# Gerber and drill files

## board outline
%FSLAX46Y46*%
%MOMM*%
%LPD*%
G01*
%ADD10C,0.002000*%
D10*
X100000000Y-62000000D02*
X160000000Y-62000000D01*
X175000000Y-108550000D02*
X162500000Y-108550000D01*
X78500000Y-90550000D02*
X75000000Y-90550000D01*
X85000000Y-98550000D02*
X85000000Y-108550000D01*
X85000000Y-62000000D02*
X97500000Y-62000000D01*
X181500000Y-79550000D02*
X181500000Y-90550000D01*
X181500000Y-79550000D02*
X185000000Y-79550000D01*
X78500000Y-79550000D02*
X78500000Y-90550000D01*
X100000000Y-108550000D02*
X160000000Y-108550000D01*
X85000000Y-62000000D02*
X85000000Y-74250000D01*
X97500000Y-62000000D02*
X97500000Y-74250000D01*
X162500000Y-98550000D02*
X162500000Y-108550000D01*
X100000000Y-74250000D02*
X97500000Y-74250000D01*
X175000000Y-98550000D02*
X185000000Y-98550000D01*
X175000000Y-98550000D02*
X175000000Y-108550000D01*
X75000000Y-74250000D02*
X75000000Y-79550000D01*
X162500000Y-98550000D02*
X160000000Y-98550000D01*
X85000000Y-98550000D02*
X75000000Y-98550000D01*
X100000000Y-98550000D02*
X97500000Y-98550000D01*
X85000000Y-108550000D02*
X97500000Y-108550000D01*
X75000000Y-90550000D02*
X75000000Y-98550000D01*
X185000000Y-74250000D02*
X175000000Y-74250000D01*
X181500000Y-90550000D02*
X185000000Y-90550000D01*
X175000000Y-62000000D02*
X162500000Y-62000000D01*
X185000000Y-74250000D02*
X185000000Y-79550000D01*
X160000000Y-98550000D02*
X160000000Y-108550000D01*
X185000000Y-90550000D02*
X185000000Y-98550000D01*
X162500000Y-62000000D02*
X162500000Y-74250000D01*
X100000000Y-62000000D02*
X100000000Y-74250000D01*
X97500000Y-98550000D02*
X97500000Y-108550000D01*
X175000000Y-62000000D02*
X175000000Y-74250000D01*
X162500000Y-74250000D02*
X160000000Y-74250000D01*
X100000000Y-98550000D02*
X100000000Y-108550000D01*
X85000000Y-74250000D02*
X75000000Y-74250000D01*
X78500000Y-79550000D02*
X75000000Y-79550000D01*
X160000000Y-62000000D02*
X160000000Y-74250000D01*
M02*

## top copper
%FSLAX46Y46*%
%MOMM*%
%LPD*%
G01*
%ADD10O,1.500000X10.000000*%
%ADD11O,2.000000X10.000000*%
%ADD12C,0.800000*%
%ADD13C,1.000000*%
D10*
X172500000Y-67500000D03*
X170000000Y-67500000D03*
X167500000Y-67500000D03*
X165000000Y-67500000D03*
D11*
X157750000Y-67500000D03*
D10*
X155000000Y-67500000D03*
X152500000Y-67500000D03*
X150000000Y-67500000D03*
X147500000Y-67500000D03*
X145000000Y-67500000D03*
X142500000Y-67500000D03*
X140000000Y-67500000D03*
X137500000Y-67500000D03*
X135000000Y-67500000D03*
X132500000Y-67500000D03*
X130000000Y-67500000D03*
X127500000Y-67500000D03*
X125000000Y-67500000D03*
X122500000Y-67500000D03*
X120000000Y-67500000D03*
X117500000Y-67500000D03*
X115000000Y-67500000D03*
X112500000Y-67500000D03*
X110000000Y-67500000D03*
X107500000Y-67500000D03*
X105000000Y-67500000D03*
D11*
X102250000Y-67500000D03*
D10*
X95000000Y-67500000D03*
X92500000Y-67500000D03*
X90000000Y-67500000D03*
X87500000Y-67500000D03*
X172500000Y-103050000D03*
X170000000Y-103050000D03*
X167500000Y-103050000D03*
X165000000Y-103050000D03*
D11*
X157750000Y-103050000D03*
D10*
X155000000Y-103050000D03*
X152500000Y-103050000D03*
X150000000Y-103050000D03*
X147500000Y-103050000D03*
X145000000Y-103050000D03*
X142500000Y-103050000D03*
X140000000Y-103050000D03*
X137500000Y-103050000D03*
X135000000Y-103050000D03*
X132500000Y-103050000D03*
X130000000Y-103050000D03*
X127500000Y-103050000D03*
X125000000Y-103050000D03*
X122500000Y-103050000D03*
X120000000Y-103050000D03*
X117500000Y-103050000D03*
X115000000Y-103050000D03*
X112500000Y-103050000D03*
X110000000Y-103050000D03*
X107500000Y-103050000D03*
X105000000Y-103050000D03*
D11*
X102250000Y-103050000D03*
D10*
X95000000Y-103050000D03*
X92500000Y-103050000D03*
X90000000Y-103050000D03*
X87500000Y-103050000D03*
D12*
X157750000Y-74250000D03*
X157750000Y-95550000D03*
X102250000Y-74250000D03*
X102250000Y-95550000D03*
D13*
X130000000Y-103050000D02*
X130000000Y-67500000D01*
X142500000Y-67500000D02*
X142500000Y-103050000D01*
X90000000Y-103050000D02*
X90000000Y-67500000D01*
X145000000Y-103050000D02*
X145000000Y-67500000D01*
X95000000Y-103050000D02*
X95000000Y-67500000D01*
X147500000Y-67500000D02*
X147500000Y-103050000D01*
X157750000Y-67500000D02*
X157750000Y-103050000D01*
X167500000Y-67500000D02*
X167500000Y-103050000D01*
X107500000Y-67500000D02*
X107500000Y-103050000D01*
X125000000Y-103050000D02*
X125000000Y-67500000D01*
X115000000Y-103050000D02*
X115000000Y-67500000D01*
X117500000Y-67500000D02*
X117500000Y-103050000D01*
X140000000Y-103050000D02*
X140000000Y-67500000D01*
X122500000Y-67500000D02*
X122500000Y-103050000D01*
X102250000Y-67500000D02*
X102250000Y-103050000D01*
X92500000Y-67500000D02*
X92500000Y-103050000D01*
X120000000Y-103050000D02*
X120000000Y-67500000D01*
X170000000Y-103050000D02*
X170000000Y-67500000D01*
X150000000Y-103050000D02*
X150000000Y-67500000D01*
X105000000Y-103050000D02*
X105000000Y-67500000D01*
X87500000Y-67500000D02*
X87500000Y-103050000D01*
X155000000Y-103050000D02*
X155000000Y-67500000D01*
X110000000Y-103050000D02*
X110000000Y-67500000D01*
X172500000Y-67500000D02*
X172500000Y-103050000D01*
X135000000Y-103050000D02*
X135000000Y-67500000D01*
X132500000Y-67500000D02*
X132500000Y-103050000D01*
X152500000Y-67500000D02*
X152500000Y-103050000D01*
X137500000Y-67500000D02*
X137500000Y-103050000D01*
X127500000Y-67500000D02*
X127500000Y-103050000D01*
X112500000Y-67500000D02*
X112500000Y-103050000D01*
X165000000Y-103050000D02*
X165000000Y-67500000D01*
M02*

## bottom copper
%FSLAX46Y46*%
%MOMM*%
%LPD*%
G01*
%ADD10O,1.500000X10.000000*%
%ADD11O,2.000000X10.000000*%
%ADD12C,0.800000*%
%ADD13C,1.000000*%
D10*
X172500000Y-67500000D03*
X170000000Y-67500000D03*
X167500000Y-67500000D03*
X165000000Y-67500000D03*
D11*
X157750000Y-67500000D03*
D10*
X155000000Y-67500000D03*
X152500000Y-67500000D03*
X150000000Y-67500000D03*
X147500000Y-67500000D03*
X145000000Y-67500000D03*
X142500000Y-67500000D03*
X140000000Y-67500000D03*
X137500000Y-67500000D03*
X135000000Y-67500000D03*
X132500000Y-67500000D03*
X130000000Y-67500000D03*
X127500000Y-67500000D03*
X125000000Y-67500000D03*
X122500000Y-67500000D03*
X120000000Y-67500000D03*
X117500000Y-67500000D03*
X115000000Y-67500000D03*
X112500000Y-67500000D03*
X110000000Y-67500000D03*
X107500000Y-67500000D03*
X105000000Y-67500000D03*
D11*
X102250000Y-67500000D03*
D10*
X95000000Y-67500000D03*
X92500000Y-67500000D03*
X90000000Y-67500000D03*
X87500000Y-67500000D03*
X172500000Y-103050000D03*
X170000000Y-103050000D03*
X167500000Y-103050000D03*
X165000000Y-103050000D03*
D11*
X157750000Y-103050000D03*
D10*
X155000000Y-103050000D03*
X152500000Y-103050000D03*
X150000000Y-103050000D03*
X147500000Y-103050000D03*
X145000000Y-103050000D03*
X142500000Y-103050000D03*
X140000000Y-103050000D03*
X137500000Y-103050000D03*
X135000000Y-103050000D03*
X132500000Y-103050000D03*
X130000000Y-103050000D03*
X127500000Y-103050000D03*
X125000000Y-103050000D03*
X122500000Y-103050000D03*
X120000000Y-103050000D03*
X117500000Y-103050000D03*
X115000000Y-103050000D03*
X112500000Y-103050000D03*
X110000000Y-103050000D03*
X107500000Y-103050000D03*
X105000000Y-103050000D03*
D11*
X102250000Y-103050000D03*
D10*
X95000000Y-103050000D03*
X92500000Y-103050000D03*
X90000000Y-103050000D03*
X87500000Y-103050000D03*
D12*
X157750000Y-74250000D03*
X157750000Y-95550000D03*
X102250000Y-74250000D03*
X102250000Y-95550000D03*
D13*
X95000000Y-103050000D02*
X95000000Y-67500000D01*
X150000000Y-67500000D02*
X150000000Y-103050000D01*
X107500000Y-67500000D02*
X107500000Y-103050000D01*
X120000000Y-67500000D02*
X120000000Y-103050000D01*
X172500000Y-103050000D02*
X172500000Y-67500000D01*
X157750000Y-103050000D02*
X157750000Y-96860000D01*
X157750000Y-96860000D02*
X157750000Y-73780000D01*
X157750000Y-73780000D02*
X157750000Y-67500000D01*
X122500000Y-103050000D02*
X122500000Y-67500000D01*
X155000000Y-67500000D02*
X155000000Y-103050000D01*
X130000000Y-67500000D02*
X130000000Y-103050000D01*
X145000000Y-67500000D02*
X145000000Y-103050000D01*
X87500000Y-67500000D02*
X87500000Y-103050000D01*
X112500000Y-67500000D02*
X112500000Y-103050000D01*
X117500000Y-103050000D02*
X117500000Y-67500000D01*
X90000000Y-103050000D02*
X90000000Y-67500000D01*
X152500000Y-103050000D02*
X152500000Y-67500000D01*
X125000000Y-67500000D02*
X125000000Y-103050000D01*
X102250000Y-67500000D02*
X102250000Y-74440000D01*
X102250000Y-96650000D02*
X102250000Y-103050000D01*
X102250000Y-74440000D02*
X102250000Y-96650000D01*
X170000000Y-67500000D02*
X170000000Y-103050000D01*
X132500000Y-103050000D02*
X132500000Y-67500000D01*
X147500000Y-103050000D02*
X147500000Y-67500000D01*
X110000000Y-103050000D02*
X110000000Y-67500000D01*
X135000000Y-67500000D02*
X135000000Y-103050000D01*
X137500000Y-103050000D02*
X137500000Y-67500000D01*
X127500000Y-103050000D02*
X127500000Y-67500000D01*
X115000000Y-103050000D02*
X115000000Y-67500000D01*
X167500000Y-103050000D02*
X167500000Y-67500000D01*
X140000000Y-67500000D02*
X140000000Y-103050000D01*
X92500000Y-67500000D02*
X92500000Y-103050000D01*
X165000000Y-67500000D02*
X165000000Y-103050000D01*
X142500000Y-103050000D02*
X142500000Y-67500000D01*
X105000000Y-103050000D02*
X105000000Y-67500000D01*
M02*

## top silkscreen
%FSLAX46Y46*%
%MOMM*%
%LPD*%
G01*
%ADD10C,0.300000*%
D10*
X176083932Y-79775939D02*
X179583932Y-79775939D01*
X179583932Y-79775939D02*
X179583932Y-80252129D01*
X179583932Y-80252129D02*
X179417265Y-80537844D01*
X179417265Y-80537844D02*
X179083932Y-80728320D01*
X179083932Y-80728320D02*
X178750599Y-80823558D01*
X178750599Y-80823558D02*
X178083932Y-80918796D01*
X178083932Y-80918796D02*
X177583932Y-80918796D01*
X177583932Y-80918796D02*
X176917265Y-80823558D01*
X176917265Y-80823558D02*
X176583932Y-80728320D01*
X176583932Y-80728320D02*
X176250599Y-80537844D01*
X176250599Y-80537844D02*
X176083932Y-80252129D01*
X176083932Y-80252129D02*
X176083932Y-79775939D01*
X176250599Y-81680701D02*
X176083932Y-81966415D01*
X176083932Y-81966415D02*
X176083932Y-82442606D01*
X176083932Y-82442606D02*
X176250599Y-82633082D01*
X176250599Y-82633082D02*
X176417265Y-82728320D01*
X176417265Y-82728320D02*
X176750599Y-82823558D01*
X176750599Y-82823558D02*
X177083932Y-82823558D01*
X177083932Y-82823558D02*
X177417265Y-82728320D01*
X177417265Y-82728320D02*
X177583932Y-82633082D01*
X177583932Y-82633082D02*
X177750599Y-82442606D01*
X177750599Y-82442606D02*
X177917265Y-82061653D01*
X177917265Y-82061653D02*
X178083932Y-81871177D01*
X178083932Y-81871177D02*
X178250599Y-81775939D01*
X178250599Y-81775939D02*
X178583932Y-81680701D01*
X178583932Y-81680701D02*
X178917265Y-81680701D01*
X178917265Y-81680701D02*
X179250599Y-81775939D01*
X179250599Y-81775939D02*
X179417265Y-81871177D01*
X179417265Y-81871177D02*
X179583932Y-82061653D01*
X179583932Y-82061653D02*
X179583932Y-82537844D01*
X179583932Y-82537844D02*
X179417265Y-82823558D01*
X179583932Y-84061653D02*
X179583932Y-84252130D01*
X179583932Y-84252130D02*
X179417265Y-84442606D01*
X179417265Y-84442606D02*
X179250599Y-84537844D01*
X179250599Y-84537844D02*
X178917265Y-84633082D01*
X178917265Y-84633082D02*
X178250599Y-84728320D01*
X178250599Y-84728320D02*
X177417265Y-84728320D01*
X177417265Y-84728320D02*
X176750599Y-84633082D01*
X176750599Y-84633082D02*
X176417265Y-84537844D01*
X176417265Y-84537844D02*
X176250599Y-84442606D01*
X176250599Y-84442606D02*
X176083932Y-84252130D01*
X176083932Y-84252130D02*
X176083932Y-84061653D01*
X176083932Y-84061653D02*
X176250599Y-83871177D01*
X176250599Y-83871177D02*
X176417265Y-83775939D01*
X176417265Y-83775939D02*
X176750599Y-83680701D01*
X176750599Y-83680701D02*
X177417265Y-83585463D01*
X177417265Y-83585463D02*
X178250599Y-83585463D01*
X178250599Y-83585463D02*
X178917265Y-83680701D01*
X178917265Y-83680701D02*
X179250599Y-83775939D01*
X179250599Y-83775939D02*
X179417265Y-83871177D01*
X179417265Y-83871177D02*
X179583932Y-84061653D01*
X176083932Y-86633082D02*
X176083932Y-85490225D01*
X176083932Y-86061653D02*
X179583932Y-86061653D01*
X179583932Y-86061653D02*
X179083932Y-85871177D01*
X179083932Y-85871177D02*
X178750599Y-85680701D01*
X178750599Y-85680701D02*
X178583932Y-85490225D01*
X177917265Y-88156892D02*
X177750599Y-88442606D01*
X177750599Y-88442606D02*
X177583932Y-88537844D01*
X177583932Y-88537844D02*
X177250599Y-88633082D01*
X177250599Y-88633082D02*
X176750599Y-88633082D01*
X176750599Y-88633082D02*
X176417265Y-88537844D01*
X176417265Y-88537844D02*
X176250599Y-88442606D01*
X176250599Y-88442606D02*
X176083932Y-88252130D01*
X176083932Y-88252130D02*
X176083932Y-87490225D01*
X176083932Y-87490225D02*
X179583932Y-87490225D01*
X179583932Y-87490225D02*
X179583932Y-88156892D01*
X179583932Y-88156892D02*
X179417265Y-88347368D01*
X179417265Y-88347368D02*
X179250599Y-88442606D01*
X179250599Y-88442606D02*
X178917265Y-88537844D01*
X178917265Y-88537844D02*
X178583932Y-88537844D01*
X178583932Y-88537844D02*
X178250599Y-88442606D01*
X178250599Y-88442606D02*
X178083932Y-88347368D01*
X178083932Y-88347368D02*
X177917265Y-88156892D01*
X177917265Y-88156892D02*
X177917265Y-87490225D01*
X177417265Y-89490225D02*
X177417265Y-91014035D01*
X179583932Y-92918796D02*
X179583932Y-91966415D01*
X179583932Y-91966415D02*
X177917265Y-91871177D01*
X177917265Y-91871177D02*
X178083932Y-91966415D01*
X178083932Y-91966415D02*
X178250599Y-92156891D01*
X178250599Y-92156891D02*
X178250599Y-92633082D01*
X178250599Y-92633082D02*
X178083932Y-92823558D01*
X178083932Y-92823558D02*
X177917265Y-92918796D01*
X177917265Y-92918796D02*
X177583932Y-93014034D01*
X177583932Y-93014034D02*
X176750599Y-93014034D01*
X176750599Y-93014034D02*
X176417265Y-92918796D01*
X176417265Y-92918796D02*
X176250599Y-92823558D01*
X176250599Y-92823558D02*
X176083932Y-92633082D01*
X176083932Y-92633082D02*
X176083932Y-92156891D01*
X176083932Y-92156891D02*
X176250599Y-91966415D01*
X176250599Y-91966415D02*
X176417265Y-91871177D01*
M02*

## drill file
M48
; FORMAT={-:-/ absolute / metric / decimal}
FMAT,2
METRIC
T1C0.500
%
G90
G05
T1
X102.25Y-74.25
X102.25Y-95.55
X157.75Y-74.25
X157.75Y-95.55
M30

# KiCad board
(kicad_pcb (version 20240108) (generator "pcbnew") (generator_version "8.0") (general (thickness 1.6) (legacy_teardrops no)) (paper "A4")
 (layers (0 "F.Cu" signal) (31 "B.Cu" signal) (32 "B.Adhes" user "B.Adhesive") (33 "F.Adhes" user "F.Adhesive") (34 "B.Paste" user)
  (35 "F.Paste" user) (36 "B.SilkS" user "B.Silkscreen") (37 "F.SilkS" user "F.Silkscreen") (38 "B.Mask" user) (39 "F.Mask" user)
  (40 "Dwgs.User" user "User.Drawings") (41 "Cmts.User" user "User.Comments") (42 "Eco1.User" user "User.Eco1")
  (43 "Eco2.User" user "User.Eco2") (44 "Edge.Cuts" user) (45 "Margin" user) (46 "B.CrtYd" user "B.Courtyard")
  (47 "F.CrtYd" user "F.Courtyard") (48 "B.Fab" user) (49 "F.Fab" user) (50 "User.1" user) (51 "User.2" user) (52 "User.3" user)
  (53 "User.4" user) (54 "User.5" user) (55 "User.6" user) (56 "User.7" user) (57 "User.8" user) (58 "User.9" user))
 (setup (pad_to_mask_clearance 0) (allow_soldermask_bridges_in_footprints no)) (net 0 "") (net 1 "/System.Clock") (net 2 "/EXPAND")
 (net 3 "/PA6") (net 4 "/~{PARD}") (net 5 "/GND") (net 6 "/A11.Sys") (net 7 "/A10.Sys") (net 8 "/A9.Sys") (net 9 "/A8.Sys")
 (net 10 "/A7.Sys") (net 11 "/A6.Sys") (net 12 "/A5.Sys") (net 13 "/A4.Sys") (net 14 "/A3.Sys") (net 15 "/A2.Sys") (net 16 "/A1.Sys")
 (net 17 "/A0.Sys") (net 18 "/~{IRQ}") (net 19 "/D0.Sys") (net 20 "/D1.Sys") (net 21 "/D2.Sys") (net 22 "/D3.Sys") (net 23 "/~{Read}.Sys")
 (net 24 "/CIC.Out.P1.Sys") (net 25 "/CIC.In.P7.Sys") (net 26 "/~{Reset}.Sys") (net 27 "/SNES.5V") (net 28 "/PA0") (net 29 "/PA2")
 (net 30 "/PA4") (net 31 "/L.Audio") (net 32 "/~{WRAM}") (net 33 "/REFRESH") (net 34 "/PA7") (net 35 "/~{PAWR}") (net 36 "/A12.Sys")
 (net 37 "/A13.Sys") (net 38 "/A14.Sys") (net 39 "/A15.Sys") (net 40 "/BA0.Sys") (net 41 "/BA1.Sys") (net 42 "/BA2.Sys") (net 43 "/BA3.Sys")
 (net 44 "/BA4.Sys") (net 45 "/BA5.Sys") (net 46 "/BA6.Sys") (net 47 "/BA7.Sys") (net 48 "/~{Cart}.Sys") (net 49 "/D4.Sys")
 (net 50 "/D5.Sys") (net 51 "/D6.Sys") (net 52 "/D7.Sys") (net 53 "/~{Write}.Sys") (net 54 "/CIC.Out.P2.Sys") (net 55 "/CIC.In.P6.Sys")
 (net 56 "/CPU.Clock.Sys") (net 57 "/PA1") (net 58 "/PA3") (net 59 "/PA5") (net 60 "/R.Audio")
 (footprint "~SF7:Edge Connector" (layer "F.Cu") (at 130 67.5)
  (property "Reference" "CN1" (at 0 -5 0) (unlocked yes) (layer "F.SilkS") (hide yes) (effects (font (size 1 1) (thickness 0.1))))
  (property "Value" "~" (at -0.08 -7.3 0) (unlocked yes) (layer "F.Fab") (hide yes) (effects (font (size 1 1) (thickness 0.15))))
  (pad "1" smd oval (at 42.5 0) (size 1.5 10) (layers "B.Cu" "B.Mask") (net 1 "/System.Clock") (thermal_bridge_angle 45))
  (pad "2" smd oval (at 40 0) (size 1.5 10) (layers "B.Cu" "B.Mask") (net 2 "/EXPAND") (thermal_bridge_angle 45))
  (pad "3" smd oval (at 37.5 0) (size 1.5 10) (layers "B.Cu" "B.Mask") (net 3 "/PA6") (thermal_bridge_angle 45))
  (pad "4" smd oval (at 35 0) (size 1.5 10) (layers "B.Cu" "B.Mask") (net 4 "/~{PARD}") (thermal_bridge_angle 45))
  (pad "5" smd oval (at 27.75 0) (size 2 10) (layers "B.Cu" "B.Mask") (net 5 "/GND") (thermal_bridge_angle 45))
  (pad "6" smd oval (at 25 0) (size 1.5 10) (layers "B.Cu" "B.Mask") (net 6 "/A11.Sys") (thermal_bridge_angle 45))
  (pad "7" smd oval (at 22.5 0) (size 1.5 10) (layers "B.Cu" "B.Mask") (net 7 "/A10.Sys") (thermal_bridge_angle 45))
  (pad "8" smd oval (at 20 0) (size 1.5 10) (layers "B.Cu" "B.Mask") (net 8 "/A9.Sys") (thermal_bridge_angle 45))
  (pad "9" smd oval (at 17.5 0) (size 1.5 10) (layers "B.Cu" "B.Mask") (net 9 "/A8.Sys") (thermal_bridge_angle 45))
  (pad "10" smd oval (at 15 0) (size 1.5 10) (layers "B.Cu" "B.Mask") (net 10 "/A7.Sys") (thermal_bridge_angle 45))
  (pad "11" smd oval (at 12.5 0) (size 1.5 10) (layers "B.Cu" "B.Mask") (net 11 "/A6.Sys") (thermal_bridge_angle 45))
  (pad "12" smd oval (at 10 0) (size 1.5 10) (layers "B.Cu" "B.Mask") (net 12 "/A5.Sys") (thermal_bridge_angle 45))
  (pad "13" smd oval (at 7.5 0) (size 1.5 10) (layers "B.Cu" "B.Mask") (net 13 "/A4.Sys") (thermal_bridge_angle 45))
  (pad "14" smd oval (at 5 0) (size 1.5 10) (layers "B.Cu" "B.Mask") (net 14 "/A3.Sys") (thermal_bridge_angle 45))
  (pad "15" smd oval (at 2.5 0) (size 1.5 10) (layers "B.Cu" "B.Mask") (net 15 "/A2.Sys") (thermal_bridge_angle 45))
  (pad "16" smd oval (at 0 0) (size 1.5 10) (layers "B.Cu" "B.Mask") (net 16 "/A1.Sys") (thermal_bridge_angle 45))
  (pad "17" smd oval (at -2.5 0) (size 1.5 10) (layers "B.Cu" "B.Mask") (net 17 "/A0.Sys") (thermal_bridge_angle 45))
  (pad "18" smd oval (at -5 0) (size 1.5 10) (layers "B.Cu" "B.Mask") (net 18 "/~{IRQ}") (thermal_bridge_angle 45))
  (pad "19" smd oval (at -7.5 0) (size 1.5 10) (layers "B.Cu" "B.Mask") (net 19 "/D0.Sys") (thermal_bridge_angle 45))
  (pad "20" smd oval (at -10 0) (size 1.5 10) (layers "B.Cu" "B.Mask") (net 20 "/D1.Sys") (thermal_bridge_angle 45))
  (pad "21" smd oval (at -12.5 0) (size 1.5 10) (layers "B.Cu" "B.Mask") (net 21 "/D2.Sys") (thermal_bridge_angle 45))
  (pad "22" smd oval (at -15 0) (size 1.5 10) (layers "B.Cu" "B.Mask") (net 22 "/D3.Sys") (thermal_bridge_angle 45))
  (pad "23" smd oval (at -17.5 0) (size 1.5 10) (layers "B.Cu" "B.Mask") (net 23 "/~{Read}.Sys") (thermal_bridge_angle 45))
  (pad "24" smd oval (at -20 0) (size 1.5 10) (layers "B.Cu" "B.Mask") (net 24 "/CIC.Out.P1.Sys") (thermal_bridge_angle 45))
  (pad "25" smd oval (at -22.5 0) (size 1.5 10) (layers "B.Cu" "B.Mask") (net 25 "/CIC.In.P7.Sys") (thermal_bridge_angle 45))
  (pad "26" smd oval (at -25 0) (size 1.5 10) (layers "B.Cu" "B.Mask") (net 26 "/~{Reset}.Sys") (thermal_bridge_angle 45))
  (pad "27" smd oval (at -27.75 0) (size 2 10) (layers "B.Cu" "B.Mask") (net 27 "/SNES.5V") (thermal_bridge_angle 45))
  (pad "28" smd oval (at -35 0) (size 1.5 10) (layers "B.Cu" "B.Mask") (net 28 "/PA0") (thermal_bridge_angle 45))
  (pad "29" smd oval (at -37.5 0) (size 1.5 10) (layers "B.Cu" "B.Mask") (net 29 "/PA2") (thermal_bridge_angle 45))
  (pad "30" smd oval (at -40 0) (size 1.5 10) (layers "B.Cu" "B.Mask") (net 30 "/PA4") (thermal_bridge_angle 45))
  (pad "31" smd oval (at -42.5 0) (size 1.5 10) (layers "B.Cu" "B.Mask") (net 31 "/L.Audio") (thermal_bridge_angle 45))
  (pad "32" smd oval (at 42.5 0) (size 1.5 10) (layers "F.Cu" "F.Mask") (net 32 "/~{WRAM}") (thermal_bridge_angle 45))
  (pad "33" smd oval (at 40 0) (size 1.5 10) (layers "F.Cu" "F.Mask") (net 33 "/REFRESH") (thermal_bridge_angle 45))
  (pad "34" smd oval (at 37.5 0) (size 1.5 10) (layers "F.Cu" "F.Mask") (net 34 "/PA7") (thermal_bridge_angle 45))
  (pad "35" smd oval (at 35 0) (size 1.5 10) (layers "F.Cu" "F.Mask") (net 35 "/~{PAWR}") (thermal_bridge_angle 45))
  (pad "36" smd oval (at 27.75 0) (size 2 10) (layers "F.Cu" "F.Mask") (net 5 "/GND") (thermal_bridge_angle 45))
  (pad "37" smd oval (at 25 0) (size 1.5 10) (layers "F.Cu" "F.Mask") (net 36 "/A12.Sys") (thermal_bridge_angle 45))
  (pad "38" smd oval (at 22.5 0) (size 1.5 10) (layers "F.Cu" "F.Mask") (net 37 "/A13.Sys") (thermal_bridge_angle 45))
  (pad "39" smd oval (at 20 0) (size 1.5 10) (layers "F.Cu" "F.Mask") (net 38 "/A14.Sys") (thermal_bridge_angle 45))
  (pad "40" smd oval (at 17.5 0) (size 1.5 10) (layers "F.Cu" "F.Mask") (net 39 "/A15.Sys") (thermal_bridge_angle 45))
  (pad "41" smd oval (at 15 0) (size 1.5 10) (layers "F.Cu" "F.Mask") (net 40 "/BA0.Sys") (thermal_bridge_angle 45))
  (pad "42" smd oval (at 12.5 0) (size 1.5 10) (layers "F.Cu" "F.Mask") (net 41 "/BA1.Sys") (thermal_bridge_angle 45))
  (pad "43" smd oval (at 10 0) (size 1.5 10) (layers "F.Cu" "F.Mask") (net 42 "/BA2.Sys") (thermal_bridge_angle 45))
  (pad "44" smd oval (at 7.5 0) (size 1.5 10) (layers "F.Cu" "F.Mask") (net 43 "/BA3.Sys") (thermal_bridge_angle 45))
  (pad "45" smd oval (at 5 0) (size 1.5 10) (layers "F.Cu" "F.Mask") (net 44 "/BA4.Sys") (thermal_bridge_angle 45))
  (pad "46" smd oval (at 2.5 0) (size 1.5 10) (layers "F.Cu" "F.Mask") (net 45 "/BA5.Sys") (thermal_bridge_angle 45))
  (pad "47" smd oval (at 0 0) (size 1.5 10) (layers "F.Cu" "F.Mask") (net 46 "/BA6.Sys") (thermal_bridge_angle 45))
  (pad "48" smd oval (at -2.5 0) (size 1.5 10) (layers "F.Cu" "F.Mask") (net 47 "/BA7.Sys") (thermal_bridge_angle 45))
  (pad "49" smd oval (at -5 0) (size 1.5 10) (layers "F.Cu" "F.Mask") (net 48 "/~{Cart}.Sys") (thermal_bridge_angle 45))
  (pad "50" smd oval (at -7.5 0) (size 1.5 10) (layers "F.Cu" "F.Mask") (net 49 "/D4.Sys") (thermal_bridge_angle 45))
  (pad "51" smd oval (at -10 0) (size 1.5 10) (layers "F.Cu" "F.Mask") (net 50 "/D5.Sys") (thermal_bridge_angle 45))
  (pad "52" smd oval (at -12.5 0) (size 1.5 10) (layers "F.Cu" "F.Mask") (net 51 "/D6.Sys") (thermal_bridge_angle 45))
  (pad "53" smd oval (at -15 0) (size 1.5 10) (layers "F.Cu" "F.Mask") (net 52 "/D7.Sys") (thermal_bridge_angle 45))
  (pad "54" smd oval (at -17.5 0) (size 1.5 10) (layers "F.Cu" "F.Mask") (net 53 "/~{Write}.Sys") (thermal_bridge_angle 45))
  (pad "55" smd oval (at -20 0) (size 1.5 10) (layers "F.Cu" "F.Mask") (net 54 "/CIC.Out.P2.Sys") (thermal_bridge_angle 45))
  (pad "56" smd oval (at -22.5 0) (size 1.5 10) (layers "F.Cu" "F.Mask") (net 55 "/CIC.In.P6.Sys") (thermal_bridge_angle 45))
  (pad "57" smd oval (at -25 0) (size 1.5 10) (layers "F.Cu" "F.Mask") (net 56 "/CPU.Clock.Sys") (thermal_bridge_angle 45))
  (pad "58" smd oval (at -27.75 0) (size 2 10) (layers "F.Cu" "F.Mask") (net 27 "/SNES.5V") (thermal_bridge_angle 45))
  (pad "59" smd oval (at -35 0) (size 1.5 10) (layers "F.Cu" "F.Mask") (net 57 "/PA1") (thermal_bridge_angle 45))
  (pad "60" smd oval (at -37.5 0) (size 1.5 10) (layers "F.Cu" "F.Mask") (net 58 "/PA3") (thermal_bridge_angle 45))
  (pad "61" smd oval (at -40 0) (size 1.5 10) (layers "F.Cu" "F.Mask") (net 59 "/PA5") (thermal_bridge_angle 45))
  (pad "62" smd oval (at -42.5 0) (size 1.5 10) (layers "F.Cu" "F.Mask") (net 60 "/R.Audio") (thermal_bridge_angle 45)))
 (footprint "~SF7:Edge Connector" (layer "F.Cu") (at 130 103.05)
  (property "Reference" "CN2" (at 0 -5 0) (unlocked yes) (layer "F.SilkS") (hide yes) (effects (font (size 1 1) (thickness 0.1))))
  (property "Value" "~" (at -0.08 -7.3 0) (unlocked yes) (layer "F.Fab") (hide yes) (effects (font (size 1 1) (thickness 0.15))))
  (pad "1" smd oval (at 42.5 0) (size 1.5 10) (layers "B.Cu" "B.Mask") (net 1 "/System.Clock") (thermal_bridge_angle 45))
  (pad "2" smd oval (at 40 0) (size 1.5 10) (layers "B.Cu" "B.Mask") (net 2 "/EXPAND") (thermal_bridge_angle 45))
  (pad "3" smd oval (at 37.5 0) (size 1.5 10) (layers "B.Cu" "B.Mask") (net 3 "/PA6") (thermal_bridge_angle 45))
  (pad "4" smd oval (at 35 0) (size 1.5 10) (layers "B.Cu" "B.Mask") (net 4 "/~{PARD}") (thermal_bridge_angle 45))
  (pad "5" smd oval (at 27.75 0) (size 2 10) (layers "B.Cu" "B.Mask") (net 5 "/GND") (thermal_bridge_angle 45))
  (pad "6" smd oval (at 25 0) (size 1.5 10) (layers "B.Cu" "B.Mask") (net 6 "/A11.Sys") (thermal_bridge_angle 45))
  (pad "7" smd oval (at 22.5 0) (size 1.5 10) (layers "B.Cu" "B.Mask") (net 7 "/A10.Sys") (thermal_bridge_angle 45))
  (pad "8" smd oval (at 20 0) (size 1.5 10) (layers "B.Cu" "B.Mask") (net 8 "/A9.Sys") (thermal_bridge_angle 45))
  (pad "9" smd oval (at 17.5 0) (size 1.5 10) (layers "B.Cu" "B.Mask") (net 9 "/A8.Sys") (thermal_bridge_angle 45))
  (pad "10" smd oval (at 15 0) (size 1.5 10) (layers "B.Cu" "B.Mask") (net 10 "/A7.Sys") (thermal_bridge_angle 45))
  (pad "11" smd oval (at 12.5 0) (size 1.5 10) (layers "B.Cu" "B.Mask") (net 11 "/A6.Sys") (thermal_bridge_angle 45))
  (pad "12" smd oval (at 10 0) (size 1.5 10) (layers "B.Cu" "B.Mask") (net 12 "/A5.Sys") (thermal_bridge_angle 45))
  (pad "13" smd oval (at 7.5 0) (size 1.5 10) (layers "B.Cu" "B.Mask") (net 13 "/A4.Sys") (thermal_bridge_angle 45))
  (pad "14" smd oval (at 5 0) (size 1.5 10) (layers "B.Cu" "B.Mask") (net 14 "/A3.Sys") (thermal_bridge_angle 45))
  (pad "15" smd oval (at 2.5 0) (size 1.5 10) (layers "B.Cu" "B.Mask") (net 15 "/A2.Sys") (thermal_bridge_angle 45))
  (pad "16" smd oval (at 0 0) (size 1.5 10) (layers "B.Cu" "B.Mask") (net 16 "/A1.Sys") (thermal_bridge_angle 45))
  (pad "17" smd oval (at -2.5 0) (size 1.5 10) (layers "B.Cu" "B.Mask") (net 17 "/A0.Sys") (thermal_bridge_angle 45))
  (pad "18" smd oval (at -5 0) (size 1.5 10) (layers "B.Cu" "B.Mask") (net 18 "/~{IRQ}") (thermal_bridge_angle 45))
  (pad "19" smd oval (at -7.5 0) (size 1.5 10) (layers "B.Cu" "B.Mask") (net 19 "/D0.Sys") (thermal_bridge_angle 45))
  (pad "20" smd oval (at -10 0) (size 1.5 10) (layers "B.Cu" "B.Mask") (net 20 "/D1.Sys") (thermal_bridge_angle 45))
  (pad "21" smd oval (at -12.5 0) (size 1.5 10) (layers "B.Cu" "B.Mask") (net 21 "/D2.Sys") (thermal_bridge_angle 45))
  (pad "22" smd oval (at -15 0) (size 1.5 10) (layers "B.Cu" "B.Mask") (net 22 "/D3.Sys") (thermal_bridge_angle 45))
  (pad "23" smd oval (at -17.5 0) (size 1.5 10) (layers "B.Cu" "B.Mask") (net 23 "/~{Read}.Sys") (thermal_bridge_angle 45))
  (pad "24" smd oval (at -20 0) (size 1.5 10) (layers "B.Cu" "B.Mask") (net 24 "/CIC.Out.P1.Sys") (thermal_bridge_angle 45))
  (pad "25" smd oval (at -22.5 0) (size 1.5 10) (layers "B.Cu" "B.Mask") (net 25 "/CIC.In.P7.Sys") (thermal_bridge_angle 45))
  (pad "26" smd oval (at -25 0) (size 1.5 10) (layers "B.Cu" "B.Mask") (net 26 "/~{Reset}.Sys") (thermal_bridge_angle 45))
  (pad "27" smd oval (at -27.75 0) (size 2 10) (layers "B.Cu" "B.Mask") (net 27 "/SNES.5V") (thermal_bridge_angle 45))
  (pad "28" smd oval (at -35 0) (size 1.5 10) (layers "B.Cu" "B.Mask") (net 28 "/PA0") (thermal_bridge_angle 45))
  (pad "29" smd oval (at -37.5 0) (size 1.5 10) (layers "B.Cu" "B.Mask") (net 29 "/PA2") (thermal_bridge_angle 45))
  (pad "30" smd oval (at -40 0) (size 1.5 10) (layers "B.Cu" "B.Mask") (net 30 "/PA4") (thermal_bridge_angle 45))
  (pad "31" smd oval (at -42.5 0) (size 1.5 10) (layers "B.Cu" "B.Mask") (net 31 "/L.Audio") (thermal_bridge_angle 45))
  (pad "32" smd oval (at 42.5 0) (size 1.5 10) (layers "F.Cu" "F.Mask") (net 32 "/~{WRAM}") (thermal_bridge_angle 45))
  (pad "33" smd oval (at 40 0) (size 1.5 10) (layers "F.Cu" "F.Mask") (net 33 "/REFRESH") (thermal_bridge_angle 45))
  (pad "34" smd oval (at 37.5 0) (size 1.5 10) (layers "F.Cu" "F.Mask") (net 34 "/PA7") (thermal_bridge_angle 45))
  (pad "35" smd oval (at 35 0) (size 1.5 10) (layers "F.Cu" "F.Mask") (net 35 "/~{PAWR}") (thermal_bridge_angle 45))
  (pad "36" smd oval (at 27.75 0) (size 2 10) (layers "F.Cu" "F.Mask") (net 5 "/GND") (thermal_bridge_angle 45))
  (pad "37" smd oval (at 25 0) (size 1.5 10) (layers "F.Cu" "F.Mask") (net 36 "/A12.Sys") (thermal_bridge_angle 45))
  (pad "38" smd oval (at 22.5 0) (size 1.5 10) (layers "F.Cu" "F.Mask") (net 37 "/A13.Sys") (thermal_bridge_angle 45))
  (pad "39" smd oval (at 20 0) (size 1.5 10) (layers "F.Cu" "F.Mask") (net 38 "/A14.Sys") (thermal_bridge_angle 45))
  (pad "40" smd oval (at 17.5 0) (size 1.5 10) (layers "F.Cu" "F.Mask") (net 39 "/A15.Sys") (thermal_bridge_angle 45))
  (pad "41" smd oval (at 15 0) (size 1.5 10) (layers "F.Cu" "F.Mask") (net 40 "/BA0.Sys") (thermal_bridge_angle 45))
  (pad "42" smd oval (at 12.5 0) (size 1.5 10) (layers "F.Cu" "F.Mask") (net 41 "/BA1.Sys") (thermal_bridge_angle 45))
  (pad "43" smd oval (at 10 0) (size 1.5 10) (layers "F.Cu" "F.Mask") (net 42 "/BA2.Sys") (thermal_bridge_angle 45))
  (pad "44" smd oval (at 7.5 0) (size 1.5 10) (layers "F.Cu" "F.Mask") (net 43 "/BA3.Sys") (thermal_bridge_angle 45))
  (pad "45" smd oval (at 5 0) (size 1.5 10) (layers "F.Cu" "F.Mask") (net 44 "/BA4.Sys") (thermal_bridge_angle 45))
  (pad "46" smd oval (at 2.5 0) (size 1.5 10) (layers "F.Cu" "F.Mask") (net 45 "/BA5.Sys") (thermal_bridge_angle 45))
  (pad "47" smd oval (at 0 0) (size 1.5 10) (layers "F.Cu" "F.Mask") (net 46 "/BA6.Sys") (thermal_bridge_angle 45))
  (pad "48" smd oval (at -2.5 0) (size 1.5 10) (layers "F.Cu" "F.Mask") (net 47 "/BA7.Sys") (thermal_bridge_angle 45))
  (pad "49" smd oval (at -5 0) (size 1.5 10) (layers "F.Cu" "F.Mask") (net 48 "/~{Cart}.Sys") (thermal_bridge_angle 45))
  (pad "50" smd oval (at -7.5 0) (size 1.5 10) (layers "F.Cu" "F.Mask") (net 49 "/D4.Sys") (thermal_bridge_angle 45))
  (pad "51" smd oval (at -10 0) (size 1.5 10) (layers "F.Cu" "F.Mask") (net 50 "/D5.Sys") (thermal_bridge_angle 45))
  (pad "52" smd oval (at -12.5 0) (size 1.5 10) (layers "F.Cu" "F.Mask") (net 51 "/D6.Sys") (thermal_bridge_angle 45))
  (pad "53" smd oval (at -15 0) (size 1.5 10) (layers "F.Cu" "F.Mask") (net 52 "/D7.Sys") (thermal_bridge_angle 45))
  (pad "54" smd oval (at -17.5 0) (size 1.5 10) (layers "F.Cu" "F.Mask") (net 53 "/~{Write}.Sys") (thermal_bridge_angle 45))
  (pad "55" smd oval (at -20 0) (size 1.5 10) (layers "F.Cu" "F.Mask") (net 54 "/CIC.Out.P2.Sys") (thermal_bridge_angle 45))
  (pad "56" smd oval (at -22.5 0) (size 1.5 10) (layers "F.Cu" "F.Mask") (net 55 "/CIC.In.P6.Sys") (thermal_bridge_angle 45))
  (pad "57" smd oval (at -25 0) (size 1.5 10) (layers "F.Cu" "F.Mask") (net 56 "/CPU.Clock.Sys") (thermal_bridge_angle 45))
  (pad "58" smd oval (at -27.75 0) (size 2 10) (layers "F.Cu" "F.Mask") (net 27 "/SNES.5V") (thermal_bridge_angle 45))
  (pad "59" smd oval (at -35 0) (size 1.5 10) (layers "F.Cu" "F.Mask") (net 57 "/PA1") (thermal_bridge_angle 45))
  (pad "60" smd oval (at -37.5 0) (size 1.5 10) (layers "F.Cu" "F.Mask") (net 58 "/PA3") (thermal_bridge_angle 45))
  (pad "61" smd oval (at -40 0) (size 1.5 10) (layers "F.Cu" "F.Mask") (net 59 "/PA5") (thermal_bridge_angle 45))
  (pad "62" smd oval (at -42.5 0) (size 1.5 10) (layers "F.Cu" "F.Mask") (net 60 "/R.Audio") (thermal_bridge_angle 45)))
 (gr_line (start 100 62) (end 160 62) (stroke (width 0.002) (type default)) (layer "Edge.Cuts"))
 (gr_line (start 175 108.55) (end 162.5 108.55) (stroke (width 0.002) (type default)) (layer "Edge.Cuts"))
 (gr_line (start 78.5 90.55) (end 75 90.55) (stroke (width 0.002) (type default)) (layer "Edge.Cuts"))
 (gr_line (start 85 98.55) (end 85 108.55) (stroke (width 0.002) (type default)) (layer "Edge.Cuts"))
 (gr_line (start 85 62) (end 97.5 62) (stroke (width 0.002) (type default)) (layer "Edge.Cuts"))
 (gr_line (start 181.5 79.55) (end 181.5 90.55) (stroke (width 0.002) (type default)) (layer "Edge.Cuts"))
 (gr_line (start 181.5 79.55) (end 185 79.55) (stroke (width 0.002) (type default)) (layer "Edge.Cuts"))
 (gr_line (start 78.5 79.55) (end 78.5 90.55) (stroke (width 0.002) (type default)) (layer "Edge.Cuts"))
 (gr_line (start 100 108.55) (end 160 108.55) (stroke (width 0.002) (type default)) (layer "Edge.Cuts"))
 (gr_line (start 85 62) (end 85 74.25) (stroke (width 0.002) (type default)) (layer "Edge.Cuts"))
 (gr_line (start 97.5 62) (end 97.5 74.25) (stroke (width 0.002) (type default)) (layer "Edge.Cuts"))
 (gr_line (start 162.5 98.55) (end 162.5 108.55) (stroke (width 0.002) (type default)) (layer "Edge.Cuts"))
 (gr_line (start 100 74.25) (end 97.5 74.25) (stroke (width 0.002) (type default)) (layer "Edge.Cuts"))
 (gr_line (start 175 98.55) (end 185 98.55) (stroke (width 0.002) (type default)) (layer "Edge.Cuts"))
 (gr_line (start 175 98.55) (end 175 108.55) (stroke (width 0.002) (type default)) (layer "Edge.Cuts"))
 (gr_line (start 75 74.25) (end 75 79.55) (stroke (width 0.002) (type default)) (layer "Edge.Cuts"))
 (gr_line (start 162.5 98.55) (end 160 98.55) (stroke (width 0.002) (type default)) (layer "Edge.Cuts"))
 (gr_line (start 85 98.55) (end 75 98.55) (stroke (width 0.002) (type default)) (layer "Edge.Cuts"))
 (gr_line (start 100 98.55) (end 97.5 98.55) (stroke (width 0.002) (type default)) (layer "Edge.Cuts"))
 (gr_line (start 85 108.55) (end 97.5 108.55) (stroke (width 0.002) (type default)) (layer "Edge.Cuts"))
 (gr_line (start 75 90.55) (end 75 98.55) (stroke (width 0.002) (type default)) (layer "Edge.Cuts"))
 (gr_line (start 185 74.25) (end 175 74.25) (stroke (width 0.002) (type default)) (layer "Edge.Cuts"))
 (gr_line (start 181.5 90.55) (end 185 90.55) (stroke (width 0.002) (type default)) (layer "Edge.Cuts"))
 (gr_line (start 175 62) (end 162.5 62) (stroke (width 0.002) (type default)) (layer "Edge.Cuts"))
 (gr_line (start 185 74.25) (end 185 79.55) (stroke (width 0.002) (type default)) (layer "Edge.Cuts"))
 (gr_line (start 160 98.55) (end 160 108.55) (stroke (width 0.002) (type default)) (layer "Edge.Cuts"))
 (gr_line (start 185 90.55) (end 185 98.55) (stroke (width 0.002) (type default)) (layer "Edge.Cuts"))
 (gr_line (start 162.5 62) (end 162.5 74.25) (stroke (width 0.002) (type default)) (layer "Edge.Cuts"))
 (gr_line (start 100 62) (end 100 74.25) (stroke (width 0.002) (type default)) (layer "Edge.Cuts"))
 (gr_line (start 97.5 98.55) (end 97.5 108.55) (stroke (width 0.002) (type default)) (layer "Edge.Cuts"))
 (gr_line (start 175 62) (end 175 74.25) (stroke (width 0.002) (type default)) (layer "Edge.Cuts"))
 (gr_line (start 162.5 74.25) (end 160 74.25) (stroke (width 0.002) (type default)) (layer "Edge.Cuts"))
 (gr_line (start 100 98.55) (end 100 108.55) (stroke (width 0.002) (type default)) (layer "Edge.Cuts"))
 (gr_line (start 85 74.25) (end 75 74.25) (stroke (width 0.002) (type default)) (layer "Edge.Cuts"))
 (gr_line (start 78.5 79.55) (end 75 79.55) (stroke (width 0.002) (type default)) (layer "Edge.Cuts"))
 (gr_line (start 160 62) (end 160 74.25) (stroke (width 0.002) (type default)) (layer "Edge.Cuts"))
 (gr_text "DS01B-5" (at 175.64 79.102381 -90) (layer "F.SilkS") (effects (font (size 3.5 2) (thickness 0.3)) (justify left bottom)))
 (segment (start 130 103.05) (end 130 67.5) (width 1) (layer "F.Cu") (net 46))
 (segment (start 95 103.05) (end 95 67.5) (width 1) (layer "B.Cu") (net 28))
 (segment (start 142.5 67.5) (end 142.5 103.05) (width 1) (layer "F.Cu") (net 41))
 (segment (start 150 67.5) (end 150 103.05) (width 1) (layer "B.Cu") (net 8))
 (segment (start 90 103.05) (end 90 67.5) (width 1) (layer "F.Cu") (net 59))
 (segment (start 145 103.05) (end 145 67.5) (width 1) (layer "F.Cu") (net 40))
 (segment (start 95 103.05) (end 95 67.5) (width 1) (layer "F.Cu") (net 57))
 (segment (start 107.5 67.5) (end 107.5 103.05) (width 1) (layer "B.Cu") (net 25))
 (segment (start 120 67.5) (end 120 103.05) (width 1) (layer "B.Cu") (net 20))
 (segment (start 172.5 103.05) (end 172.5 67.5) (width 1) (layer "B.Cu") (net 1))
 (segment (start 147.5 67.5) (end 147.5 103.05) (width 1) (layer "F.Cu") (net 39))
 (segment (start 157.75 67.5) (end 157.75 103.05) (width 1) (layer "F.Cu") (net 5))
 (via (at 157.75 74.25) (size 0.8) (drill 0.5) (layers "F.Cu" "B.Cu") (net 5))
 (via (at 157.75 95.55) (size 0.8) (drill 0.5) (layers "F.Cu" "B.Cu") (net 5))
 (segment (start 157.75 103.05) (end 157.75 96.86) (width 1) (layer "B.Cu") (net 5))
 (segment (start 157.75 96.86) (end 157.75 73.78) (width 1) (layer "B.Cu") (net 5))
 (segment (start 157.75 73.78) (end 157.75 67.5) (width 1) (layer "B.Cu") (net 5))
 (segment (start 122.5 103.05) (end 122.5 67.5) (width 1) (layer "B.Cu") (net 19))
 (segment (start 155 67.5) (end 155 103.05) (width 1) (layer "B.Cu") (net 6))
 (segment (start 130 67.5) (end 130 103.05) (width 1) (layer "B.Cu") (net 16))
 (segment (start 145 67.5) (end 145 103.05) (width 1) (layer "B.Cu") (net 10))
 (segment (start 167.5 67.5) (end 167.5 103.05) (width 1) (layer "F.Cu") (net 34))
 (segment (start 87.5 67.5) (end 87.5 103.05) (width 1) (layer "B.Cu") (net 31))
 (segment (start 112.5 67.5) (end 112.5 103.05) (width 1) (layer "B.Cu") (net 23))
 (segment (start 107.5 67.5) (end 107.5 103.05) (width 1) (layer "F.Cu") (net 55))
 (segment (start 117.5 103.05) (end 117.5 67.5) (width 1) (layer "B.Cu") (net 21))
 (segment (start 90 103.05) (end 90 67.5) (width 1) (layer "B.Cu") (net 30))
 (segment (start 125 103.05) (end 125 67.5) (width 1) (layer "F.Cu") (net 48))
 (segment (start 115 103.05) (end 115 67.5) (width 1) (layer "F.Cu") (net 52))
 (segment (start 152.5 103.05) (end 152.5 67.5) (width 1) (layer "B.Cu") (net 7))
 (segment (start 117.5 67.5) (end 117.5 103.05) (width 1) (layer "F.Cu") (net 51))
 (segment (start 140 103.05) (end 140 67.5) (width 1) (layer "F.Cu") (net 42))
 (segment (start 125 67.5) (end 125 103.05) (width 1) (layer "B.Cu") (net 18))
 (segment (start 122.5 67.5) (end 122.5 103.05) (width 1) (layer "F.Cu") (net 49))
 (segment (start 102.25 67.5) (end 102.25 103.05) (width 1) (layer "F.Cu") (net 27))
 (via (at 102.25 74.25) (size 0.8) (drill 0.5) (layers "F.Cu" "B.Cu") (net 27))
 (via (at 102.25 95.55) (size 0.8) (drill 0.5) (layers "F.Cu" "B.Cu") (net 27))
 (segment (start 102.25 67.5) (end 102.25 74.44) (width 1) (layer "B.Cu") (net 27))
 (segment (start 102.25 96.65) (end 102.25 103.05) (width 1) (layer "B.Cu") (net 27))
 (segment (start 102.25 74.44) (end 102.25 96.65) (width 1) (layer "B.Cu") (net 27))
 (segment (start 92.5 67.5) (end 92.5 103.05) (width 1) (layer "F.Cu") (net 58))
 (segment (start 170 67.5) (end 170 103.05) (width 1) (layer "B.Cu") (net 2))
 (segment (start 132.5 103.05) (end 132.5 67.5) (width 1) (layer "B.Cu") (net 15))
 (segment (start 147.5 103.05) (end 147.5 67.5) (width 1) (layer "B.Cu") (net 9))
 (segment (start 120 103.05) (end 120 67.5) (width 1) (layer "F.Cu") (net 50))
 (segment (start 110 103.05) (end 110 67.5) (width 1) (layer "B.Cu") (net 24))
 (segment (start 135 67.5) (end 135 103.05) (width 1) (layer "B.Cu") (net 14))
 (segment (start 170 103.05) (end 170 67.5) (width 1) (layer "F.Cu") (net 33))
 (segment (start 137.5 103.05) (end 137.5 67.5) (width 1) (layer "B.Cu") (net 13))
 (segment (start 150 103.05) (end 150 67.5) (width 1) (layer "F.Cu") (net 38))
 (segment (start 127.5 103.05) (end 127.5 67.5) (width 1) (layer "B.Cu") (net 17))
 (segment (start 115 103.05) (end 115 67.5) (width 1) (layer "B.Cu") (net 22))
 (segment (start 167.5 103.05) (end 167.5 67.5) (width 1) (layer "B.Cu") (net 3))
 (segment (start 105 103.05) (end 105 67.5) (width 1) (layer "F.Cu") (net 56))
 (segment (start 87.5 67.5) (end 87.5 103.05) (width 1) (layer "F.Cu") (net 60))
 (segment (start 155 103.05) (end 155 67.5) (width 1) (layer "F.Cu") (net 36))
 (segment (start 140 67.5) (end 140 103.05) (width 1) (layer "B.Cu") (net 12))
 (segment (start 92.5 67.5) (end 92.5 103.05) (width 1) (layer "B.Cu") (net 29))
 (segment (start 165 67.5) (end 165 103.05) (width 1) (layer "B.Cu") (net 4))
 (segment (start 142.5 103.05) (end 142.5 67.5) (width 1) (layer "B.Cu") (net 11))
 (segment (start 110 103.05) (end 110 67.5) (width 1) (layer "F.Cu") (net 54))
 (segment (start 172.5 67.5) (end 172.5 103.05) (width 1) (layer "F.Cu") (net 32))
 (segment (start 135 103.05) (end 135 67.5) (width 1) (layer "F.Cu") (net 44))
 (segment (start 132.5 67.5) (end 132.5 103.05) (width 1) (layer "F.Cu") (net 45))
 (segment (start 152.5 67.5) (end 152.5 103.05) (width 1) (layer "F.Cu") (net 37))
 (segment (start 105 103.05) (end 105 67.5) (width 1) (layer "B.Cu") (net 26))
 (segment (start 137.5 67.5) (end 137.5 103.05) (width 1) (layer "F.Cu") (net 43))
 (segment (start 127.5 67.5) (end 127.5 103.05) (width 1) (layer "F.Cu") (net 47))
 (segment (start 112.5 67.5) (end 112.5 103.05) (width 1) (layer "F.Cu") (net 53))
 (segment (start 165 103.05) (end 165 67.5) (width 1) (layer "F.Cu") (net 35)))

